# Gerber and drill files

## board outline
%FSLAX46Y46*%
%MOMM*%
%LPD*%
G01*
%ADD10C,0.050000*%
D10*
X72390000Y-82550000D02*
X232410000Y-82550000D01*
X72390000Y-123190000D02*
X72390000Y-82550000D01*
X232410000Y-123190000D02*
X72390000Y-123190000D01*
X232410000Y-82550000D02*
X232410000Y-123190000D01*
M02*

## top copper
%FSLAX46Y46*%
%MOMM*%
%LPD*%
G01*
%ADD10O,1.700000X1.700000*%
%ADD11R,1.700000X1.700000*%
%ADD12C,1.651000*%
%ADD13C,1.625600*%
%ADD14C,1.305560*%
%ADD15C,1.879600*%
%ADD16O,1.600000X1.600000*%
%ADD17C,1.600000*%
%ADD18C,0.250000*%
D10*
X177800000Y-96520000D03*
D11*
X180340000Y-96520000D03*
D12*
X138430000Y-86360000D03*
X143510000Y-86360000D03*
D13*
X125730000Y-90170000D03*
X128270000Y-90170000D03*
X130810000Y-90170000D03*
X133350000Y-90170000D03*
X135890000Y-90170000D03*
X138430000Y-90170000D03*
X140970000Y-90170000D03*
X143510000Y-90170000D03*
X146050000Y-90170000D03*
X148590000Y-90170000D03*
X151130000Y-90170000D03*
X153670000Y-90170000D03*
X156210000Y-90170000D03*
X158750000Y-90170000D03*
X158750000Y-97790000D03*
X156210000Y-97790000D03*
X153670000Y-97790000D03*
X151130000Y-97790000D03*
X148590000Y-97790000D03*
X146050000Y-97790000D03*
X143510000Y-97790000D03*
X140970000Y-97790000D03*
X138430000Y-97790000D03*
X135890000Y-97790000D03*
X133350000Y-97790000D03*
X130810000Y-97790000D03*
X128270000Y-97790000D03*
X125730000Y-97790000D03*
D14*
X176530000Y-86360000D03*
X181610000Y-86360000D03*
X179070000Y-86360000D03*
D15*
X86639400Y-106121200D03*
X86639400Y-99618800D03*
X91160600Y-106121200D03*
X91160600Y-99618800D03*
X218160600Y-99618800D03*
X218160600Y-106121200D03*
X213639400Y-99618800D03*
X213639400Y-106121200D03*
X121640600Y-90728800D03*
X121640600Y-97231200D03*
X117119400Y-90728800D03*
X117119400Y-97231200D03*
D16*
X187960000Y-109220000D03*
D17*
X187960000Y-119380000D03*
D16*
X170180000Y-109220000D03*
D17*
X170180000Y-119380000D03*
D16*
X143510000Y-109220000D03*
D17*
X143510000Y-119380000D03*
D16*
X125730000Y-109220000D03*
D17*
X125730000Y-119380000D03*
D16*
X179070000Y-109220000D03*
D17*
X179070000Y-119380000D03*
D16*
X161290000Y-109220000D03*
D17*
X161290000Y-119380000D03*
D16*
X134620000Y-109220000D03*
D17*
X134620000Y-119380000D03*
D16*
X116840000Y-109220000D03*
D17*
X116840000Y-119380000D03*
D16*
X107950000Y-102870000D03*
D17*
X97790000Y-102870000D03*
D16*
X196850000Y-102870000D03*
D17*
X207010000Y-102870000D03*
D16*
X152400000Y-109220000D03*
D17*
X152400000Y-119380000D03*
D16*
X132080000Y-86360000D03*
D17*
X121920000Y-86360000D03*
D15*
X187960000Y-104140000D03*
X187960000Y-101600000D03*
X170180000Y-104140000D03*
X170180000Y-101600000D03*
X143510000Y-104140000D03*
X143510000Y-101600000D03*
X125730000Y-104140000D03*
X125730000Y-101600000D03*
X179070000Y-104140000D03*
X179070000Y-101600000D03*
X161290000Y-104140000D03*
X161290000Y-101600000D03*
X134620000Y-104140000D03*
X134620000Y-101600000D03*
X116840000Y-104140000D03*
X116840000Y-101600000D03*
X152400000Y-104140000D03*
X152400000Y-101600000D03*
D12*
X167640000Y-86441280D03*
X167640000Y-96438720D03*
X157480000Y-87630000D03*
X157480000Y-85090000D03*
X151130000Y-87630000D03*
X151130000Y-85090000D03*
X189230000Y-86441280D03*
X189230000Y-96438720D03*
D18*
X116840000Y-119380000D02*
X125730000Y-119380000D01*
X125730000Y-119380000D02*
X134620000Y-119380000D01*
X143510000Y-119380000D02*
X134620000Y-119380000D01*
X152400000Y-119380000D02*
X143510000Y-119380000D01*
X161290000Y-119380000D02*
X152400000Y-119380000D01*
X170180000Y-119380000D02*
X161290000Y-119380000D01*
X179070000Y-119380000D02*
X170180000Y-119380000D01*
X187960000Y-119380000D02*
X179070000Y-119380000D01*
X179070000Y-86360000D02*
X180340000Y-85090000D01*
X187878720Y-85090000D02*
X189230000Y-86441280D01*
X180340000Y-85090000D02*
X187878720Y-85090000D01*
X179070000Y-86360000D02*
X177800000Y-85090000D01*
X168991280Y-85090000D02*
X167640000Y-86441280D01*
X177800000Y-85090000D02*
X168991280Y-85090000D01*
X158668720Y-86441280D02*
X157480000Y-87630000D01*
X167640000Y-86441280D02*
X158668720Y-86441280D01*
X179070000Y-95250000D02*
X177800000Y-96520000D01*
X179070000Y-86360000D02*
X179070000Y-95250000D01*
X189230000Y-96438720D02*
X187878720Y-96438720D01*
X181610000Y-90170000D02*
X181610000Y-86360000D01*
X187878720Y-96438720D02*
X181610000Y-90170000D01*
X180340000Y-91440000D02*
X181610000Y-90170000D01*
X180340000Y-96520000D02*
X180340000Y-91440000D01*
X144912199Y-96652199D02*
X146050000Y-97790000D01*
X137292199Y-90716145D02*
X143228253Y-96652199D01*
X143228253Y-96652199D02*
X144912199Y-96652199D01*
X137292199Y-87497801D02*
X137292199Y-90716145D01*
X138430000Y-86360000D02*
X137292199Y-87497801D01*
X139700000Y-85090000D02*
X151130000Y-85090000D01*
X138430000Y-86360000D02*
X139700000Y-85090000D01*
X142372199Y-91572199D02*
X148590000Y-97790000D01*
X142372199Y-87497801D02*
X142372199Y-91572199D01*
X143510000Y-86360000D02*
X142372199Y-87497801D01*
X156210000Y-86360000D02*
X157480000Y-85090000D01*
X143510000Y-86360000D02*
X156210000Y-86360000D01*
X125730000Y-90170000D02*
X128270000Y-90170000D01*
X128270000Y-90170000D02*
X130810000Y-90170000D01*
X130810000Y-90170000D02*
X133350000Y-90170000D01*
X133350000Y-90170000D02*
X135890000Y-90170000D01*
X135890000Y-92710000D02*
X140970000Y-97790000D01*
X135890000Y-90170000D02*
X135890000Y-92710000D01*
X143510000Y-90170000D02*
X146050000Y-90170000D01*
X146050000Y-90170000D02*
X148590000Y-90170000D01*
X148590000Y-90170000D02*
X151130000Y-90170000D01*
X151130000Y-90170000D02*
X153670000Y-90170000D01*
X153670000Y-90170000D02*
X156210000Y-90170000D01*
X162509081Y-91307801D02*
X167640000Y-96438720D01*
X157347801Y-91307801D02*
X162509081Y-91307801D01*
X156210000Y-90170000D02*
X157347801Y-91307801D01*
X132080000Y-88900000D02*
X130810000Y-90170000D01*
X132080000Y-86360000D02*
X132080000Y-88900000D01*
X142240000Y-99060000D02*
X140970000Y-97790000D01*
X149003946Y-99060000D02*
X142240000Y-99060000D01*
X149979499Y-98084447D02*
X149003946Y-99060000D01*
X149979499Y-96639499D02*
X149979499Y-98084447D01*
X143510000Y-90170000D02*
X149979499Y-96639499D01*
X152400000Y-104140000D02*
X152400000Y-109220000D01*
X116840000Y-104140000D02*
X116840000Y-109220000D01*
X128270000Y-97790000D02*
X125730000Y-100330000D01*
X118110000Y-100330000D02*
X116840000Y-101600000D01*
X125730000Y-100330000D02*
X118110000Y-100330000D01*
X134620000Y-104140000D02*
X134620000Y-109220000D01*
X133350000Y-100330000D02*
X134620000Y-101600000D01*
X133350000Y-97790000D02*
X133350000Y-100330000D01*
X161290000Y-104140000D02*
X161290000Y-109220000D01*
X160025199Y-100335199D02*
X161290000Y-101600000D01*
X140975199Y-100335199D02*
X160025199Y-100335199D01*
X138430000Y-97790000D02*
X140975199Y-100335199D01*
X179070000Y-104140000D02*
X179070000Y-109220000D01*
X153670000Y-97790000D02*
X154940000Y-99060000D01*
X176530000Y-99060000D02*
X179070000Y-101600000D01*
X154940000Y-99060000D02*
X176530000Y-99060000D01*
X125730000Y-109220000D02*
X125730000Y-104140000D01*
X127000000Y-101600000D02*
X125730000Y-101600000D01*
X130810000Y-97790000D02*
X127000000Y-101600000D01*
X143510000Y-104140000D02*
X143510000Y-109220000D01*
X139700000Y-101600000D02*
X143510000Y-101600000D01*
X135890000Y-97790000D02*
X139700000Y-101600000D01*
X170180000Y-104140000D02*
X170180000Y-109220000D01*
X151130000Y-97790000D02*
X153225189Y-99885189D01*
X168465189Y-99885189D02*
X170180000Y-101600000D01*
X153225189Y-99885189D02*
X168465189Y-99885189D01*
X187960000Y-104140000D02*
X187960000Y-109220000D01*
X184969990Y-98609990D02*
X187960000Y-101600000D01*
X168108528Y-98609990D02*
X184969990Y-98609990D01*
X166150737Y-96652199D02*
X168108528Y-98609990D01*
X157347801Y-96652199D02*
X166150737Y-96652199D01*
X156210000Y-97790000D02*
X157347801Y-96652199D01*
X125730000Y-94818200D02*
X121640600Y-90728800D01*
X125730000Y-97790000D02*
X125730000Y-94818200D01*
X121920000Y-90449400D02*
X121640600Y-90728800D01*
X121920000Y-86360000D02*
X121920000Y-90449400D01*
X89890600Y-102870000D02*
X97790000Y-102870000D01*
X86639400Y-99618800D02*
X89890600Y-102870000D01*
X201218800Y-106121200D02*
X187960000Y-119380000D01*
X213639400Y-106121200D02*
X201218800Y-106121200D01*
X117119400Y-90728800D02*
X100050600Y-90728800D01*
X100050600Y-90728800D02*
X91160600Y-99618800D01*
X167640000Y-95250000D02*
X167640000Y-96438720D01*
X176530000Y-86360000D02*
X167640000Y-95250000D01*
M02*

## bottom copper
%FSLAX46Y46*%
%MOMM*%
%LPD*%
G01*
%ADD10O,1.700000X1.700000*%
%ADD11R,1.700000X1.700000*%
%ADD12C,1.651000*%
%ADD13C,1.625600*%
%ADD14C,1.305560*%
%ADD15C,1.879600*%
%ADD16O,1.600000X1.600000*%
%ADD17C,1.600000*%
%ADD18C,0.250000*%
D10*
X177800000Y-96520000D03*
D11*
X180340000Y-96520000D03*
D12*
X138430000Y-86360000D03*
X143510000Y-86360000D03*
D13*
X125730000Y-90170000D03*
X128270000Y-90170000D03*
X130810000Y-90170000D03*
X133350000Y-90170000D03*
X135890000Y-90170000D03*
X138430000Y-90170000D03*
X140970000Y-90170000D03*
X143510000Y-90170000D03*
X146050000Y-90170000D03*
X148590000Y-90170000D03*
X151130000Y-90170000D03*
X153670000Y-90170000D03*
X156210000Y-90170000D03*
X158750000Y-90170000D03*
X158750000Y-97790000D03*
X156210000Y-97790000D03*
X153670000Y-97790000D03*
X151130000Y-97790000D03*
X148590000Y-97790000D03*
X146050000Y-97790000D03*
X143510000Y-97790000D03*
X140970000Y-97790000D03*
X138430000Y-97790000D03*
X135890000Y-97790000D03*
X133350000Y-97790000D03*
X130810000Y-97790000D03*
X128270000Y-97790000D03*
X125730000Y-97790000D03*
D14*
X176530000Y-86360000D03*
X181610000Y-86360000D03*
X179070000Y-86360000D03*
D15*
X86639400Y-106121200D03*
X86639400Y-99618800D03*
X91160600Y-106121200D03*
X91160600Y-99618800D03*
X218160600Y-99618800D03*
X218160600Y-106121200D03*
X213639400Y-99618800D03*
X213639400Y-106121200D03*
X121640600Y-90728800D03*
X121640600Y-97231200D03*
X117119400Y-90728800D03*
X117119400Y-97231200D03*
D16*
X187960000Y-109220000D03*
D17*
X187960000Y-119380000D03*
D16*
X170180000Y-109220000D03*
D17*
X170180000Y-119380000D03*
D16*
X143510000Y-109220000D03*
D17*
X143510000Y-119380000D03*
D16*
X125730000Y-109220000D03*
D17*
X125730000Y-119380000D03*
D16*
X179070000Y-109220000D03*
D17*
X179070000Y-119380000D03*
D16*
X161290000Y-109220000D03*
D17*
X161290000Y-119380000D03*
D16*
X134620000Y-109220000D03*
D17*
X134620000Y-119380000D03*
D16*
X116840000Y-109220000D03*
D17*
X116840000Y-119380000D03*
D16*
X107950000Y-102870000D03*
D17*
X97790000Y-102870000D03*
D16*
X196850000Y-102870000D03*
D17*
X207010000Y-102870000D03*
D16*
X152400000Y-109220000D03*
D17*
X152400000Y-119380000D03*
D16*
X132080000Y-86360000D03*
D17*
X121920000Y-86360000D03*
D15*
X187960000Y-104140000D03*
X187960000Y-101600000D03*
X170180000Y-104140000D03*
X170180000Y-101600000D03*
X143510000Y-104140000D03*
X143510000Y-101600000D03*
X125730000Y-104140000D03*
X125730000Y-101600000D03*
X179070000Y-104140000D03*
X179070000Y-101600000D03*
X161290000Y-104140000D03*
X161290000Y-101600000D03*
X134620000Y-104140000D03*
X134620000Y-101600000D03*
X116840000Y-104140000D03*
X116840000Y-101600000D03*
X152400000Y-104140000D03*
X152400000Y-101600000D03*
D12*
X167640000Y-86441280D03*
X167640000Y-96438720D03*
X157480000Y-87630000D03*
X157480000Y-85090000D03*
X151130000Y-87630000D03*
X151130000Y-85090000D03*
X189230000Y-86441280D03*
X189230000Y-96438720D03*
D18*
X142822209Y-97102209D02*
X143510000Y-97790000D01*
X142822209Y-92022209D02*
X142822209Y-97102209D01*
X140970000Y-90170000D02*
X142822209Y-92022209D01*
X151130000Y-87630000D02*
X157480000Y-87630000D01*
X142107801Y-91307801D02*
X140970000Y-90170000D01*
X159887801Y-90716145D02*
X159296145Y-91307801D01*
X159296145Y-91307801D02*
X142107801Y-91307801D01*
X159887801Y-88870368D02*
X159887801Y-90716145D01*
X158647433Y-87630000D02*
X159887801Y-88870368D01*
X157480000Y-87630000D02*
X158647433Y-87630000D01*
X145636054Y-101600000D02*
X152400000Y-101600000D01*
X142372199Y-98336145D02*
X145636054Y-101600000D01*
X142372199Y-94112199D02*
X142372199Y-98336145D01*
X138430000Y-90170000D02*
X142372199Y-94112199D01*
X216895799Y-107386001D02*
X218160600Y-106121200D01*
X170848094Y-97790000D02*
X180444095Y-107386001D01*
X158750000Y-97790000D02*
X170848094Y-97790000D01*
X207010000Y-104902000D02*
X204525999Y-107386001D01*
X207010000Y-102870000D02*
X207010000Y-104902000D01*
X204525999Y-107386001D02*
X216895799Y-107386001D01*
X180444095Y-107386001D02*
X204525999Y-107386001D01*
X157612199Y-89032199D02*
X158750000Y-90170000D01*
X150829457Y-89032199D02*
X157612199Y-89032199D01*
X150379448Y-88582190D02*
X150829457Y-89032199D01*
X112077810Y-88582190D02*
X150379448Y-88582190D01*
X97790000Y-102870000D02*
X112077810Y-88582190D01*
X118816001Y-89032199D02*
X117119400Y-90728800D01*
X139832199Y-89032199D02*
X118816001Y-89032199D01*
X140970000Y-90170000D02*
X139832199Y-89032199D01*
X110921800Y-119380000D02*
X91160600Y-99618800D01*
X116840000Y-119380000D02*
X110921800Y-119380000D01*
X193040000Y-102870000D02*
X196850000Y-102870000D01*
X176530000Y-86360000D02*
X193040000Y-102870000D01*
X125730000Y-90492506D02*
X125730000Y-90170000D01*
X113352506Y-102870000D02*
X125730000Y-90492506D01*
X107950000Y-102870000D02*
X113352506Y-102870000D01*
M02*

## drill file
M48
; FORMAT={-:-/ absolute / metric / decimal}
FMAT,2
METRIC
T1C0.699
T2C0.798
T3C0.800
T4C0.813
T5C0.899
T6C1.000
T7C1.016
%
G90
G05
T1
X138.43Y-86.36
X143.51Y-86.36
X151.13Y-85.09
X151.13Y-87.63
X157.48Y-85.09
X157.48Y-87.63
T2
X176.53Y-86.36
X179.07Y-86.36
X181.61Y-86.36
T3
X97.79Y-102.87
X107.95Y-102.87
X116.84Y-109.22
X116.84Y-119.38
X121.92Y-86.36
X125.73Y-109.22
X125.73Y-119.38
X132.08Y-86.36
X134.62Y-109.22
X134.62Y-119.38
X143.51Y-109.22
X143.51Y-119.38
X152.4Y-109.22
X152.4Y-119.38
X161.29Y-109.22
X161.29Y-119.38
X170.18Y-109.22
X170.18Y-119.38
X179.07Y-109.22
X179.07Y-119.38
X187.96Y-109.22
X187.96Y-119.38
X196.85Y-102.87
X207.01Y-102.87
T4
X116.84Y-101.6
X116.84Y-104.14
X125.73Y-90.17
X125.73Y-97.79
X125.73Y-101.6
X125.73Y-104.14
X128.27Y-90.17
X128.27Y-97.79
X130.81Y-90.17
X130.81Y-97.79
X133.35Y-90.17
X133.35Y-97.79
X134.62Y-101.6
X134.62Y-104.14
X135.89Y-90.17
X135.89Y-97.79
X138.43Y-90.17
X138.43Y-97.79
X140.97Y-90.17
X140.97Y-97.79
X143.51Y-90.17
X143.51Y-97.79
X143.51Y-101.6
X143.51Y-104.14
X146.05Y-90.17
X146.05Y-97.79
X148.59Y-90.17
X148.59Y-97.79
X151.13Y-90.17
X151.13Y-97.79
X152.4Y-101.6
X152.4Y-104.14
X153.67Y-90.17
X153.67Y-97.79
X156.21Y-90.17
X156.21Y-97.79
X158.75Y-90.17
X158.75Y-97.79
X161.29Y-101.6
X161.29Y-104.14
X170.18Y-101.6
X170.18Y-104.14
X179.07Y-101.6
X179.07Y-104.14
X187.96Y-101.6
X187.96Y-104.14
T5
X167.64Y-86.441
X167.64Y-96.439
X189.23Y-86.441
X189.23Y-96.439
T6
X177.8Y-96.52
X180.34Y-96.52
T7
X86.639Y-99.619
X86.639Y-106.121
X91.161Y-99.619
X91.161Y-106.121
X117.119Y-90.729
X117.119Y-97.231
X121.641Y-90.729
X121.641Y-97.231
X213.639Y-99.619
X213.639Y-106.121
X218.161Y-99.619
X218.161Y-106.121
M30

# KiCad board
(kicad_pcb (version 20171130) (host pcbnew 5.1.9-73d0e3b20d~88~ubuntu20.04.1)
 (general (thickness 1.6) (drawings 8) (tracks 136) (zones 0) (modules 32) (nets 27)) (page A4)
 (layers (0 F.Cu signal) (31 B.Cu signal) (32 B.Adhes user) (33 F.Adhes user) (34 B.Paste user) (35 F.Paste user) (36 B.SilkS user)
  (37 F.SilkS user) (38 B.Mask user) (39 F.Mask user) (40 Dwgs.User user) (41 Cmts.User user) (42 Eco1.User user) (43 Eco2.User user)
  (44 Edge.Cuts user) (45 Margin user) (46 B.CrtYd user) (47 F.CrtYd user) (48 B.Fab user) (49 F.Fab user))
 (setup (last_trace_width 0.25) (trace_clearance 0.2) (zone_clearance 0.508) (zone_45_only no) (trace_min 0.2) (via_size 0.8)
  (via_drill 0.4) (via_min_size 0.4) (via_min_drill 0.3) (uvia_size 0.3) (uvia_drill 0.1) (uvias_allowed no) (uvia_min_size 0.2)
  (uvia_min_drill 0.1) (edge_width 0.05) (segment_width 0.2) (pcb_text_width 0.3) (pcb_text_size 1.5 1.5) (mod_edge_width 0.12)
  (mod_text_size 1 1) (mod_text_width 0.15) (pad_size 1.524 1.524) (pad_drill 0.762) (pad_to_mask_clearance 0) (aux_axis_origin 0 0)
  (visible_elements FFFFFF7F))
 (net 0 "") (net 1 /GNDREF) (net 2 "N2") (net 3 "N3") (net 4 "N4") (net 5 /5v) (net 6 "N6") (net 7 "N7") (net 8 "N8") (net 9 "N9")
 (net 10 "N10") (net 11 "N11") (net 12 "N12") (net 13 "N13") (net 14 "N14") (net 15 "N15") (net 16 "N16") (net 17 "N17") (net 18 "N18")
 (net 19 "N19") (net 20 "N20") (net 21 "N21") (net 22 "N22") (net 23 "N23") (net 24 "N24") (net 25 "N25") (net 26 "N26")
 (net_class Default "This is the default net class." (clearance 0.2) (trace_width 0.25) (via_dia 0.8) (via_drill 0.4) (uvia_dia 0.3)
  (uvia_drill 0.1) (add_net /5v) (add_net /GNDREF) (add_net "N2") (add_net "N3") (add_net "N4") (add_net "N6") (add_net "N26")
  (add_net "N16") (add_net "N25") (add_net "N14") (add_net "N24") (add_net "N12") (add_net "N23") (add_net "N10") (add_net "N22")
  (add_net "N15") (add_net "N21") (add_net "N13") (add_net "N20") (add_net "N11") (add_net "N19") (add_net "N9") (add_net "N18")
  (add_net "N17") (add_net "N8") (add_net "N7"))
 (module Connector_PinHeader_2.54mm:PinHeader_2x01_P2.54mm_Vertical (layer F.Cu) (at 180.34 96.52 180)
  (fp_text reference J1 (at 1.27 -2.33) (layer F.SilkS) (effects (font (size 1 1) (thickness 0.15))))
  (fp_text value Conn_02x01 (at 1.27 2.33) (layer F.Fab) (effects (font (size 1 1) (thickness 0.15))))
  (pad 2 thru_hole oval (at 2.54 0 180) (size 1.7 1.7) (drill 1) (layers *.Cu *.Mask) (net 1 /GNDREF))
  (pad 1 thru_hole rect (at 0 0 180) (size 1.7 1.7) (drill 1) (layers *.Cu *.Mask) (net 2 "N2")))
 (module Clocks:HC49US (layer F.Cu) (at 140.97 86.36 180)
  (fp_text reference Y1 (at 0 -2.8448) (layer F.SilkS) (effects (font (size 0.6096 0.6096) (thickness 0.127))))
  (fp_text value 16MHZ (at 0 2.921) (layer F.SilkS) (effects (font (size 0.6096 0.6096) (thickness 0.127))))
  (pad 2 thru_hole circle (at 2.54 0 180) (size 1.651 1.651) (drill 0.6985) (layers *.Cu *.Mask) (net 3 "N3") (solder_mask_margin 0.1016))
  (pad 1 thru_hole circle (at -2.54 0 180) (size 1.651 1.651) (drill 0.6985) (layers *.Cu *.Mask) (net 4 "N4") (solder_mask_margin 0.1016)))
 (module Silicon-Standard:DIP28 (layer F.Cu) (at 142.24 93.98)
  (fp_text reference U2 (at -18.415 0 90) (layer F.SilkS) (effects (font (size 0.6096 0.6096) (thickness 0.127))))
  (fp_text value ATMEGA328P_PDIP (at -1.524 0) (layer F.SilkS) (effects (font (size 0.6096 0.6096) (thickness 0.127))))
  (pad 28 thru_hole circle (at -16.51 -3.81) (size 1.6256 1.6256) (drill 0.8128) (layers *.Cu *.Mask) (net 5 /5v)
   (solder_mask_margin 0.1016))
  (pad 27 thru_hole circle (at -13.97 -3.81) (size 1.6256 1.6256) (drill 0.8128) (layers *.Cu *.Mask) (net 5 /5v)
   (solder_mask_margin 0.1016))
  (pad 26 thru_hole circle (at -11.43 -3.81) (size 1.6256 1.6256) (drill 0.8128) (layers *.Cu *.Mask) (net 5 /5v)
   (solder_mask_margin 0.1016))
  (pad 25 thru_hole circle (at -8.89 -3.81) (size 1.6256 1.6256) (drill 0.8128) (layers *.Cu *.Mask) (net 5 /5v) (solder_mask_margin 0.1016))
  (pad 24 thru_hole circle (at -6.35 -3.81) (size 1.6256 1.6256) (drill 0.8128) (layers *.Cu *.Mask) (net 5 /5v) (solder_mask_margin 0.1016))
  (pad 23 thru_hole circle (at -3.81 -3.81) (size 1.6256 1.6256) (drill 0.8128) (layers *.Cu *.Mask) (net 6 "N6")
   (solder_mask_margin 0.1016))
  (pad 22 thru_hole circle (at -1.27 -3.81) (size 1.6256 1.6256) (drill 0.8128) (layers *.Cu *.Mask) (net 1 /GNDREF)
   (solder_mask_margin 0.1016))
  (pad 21 thru_hole circle (at 1.27 -3.81) (size 1.6256 1.6256) (drill 0.8128) (layers *.Cu *.Mask) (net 5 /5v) (solder_mask_margin 0.1016))
  (pad 20 thru_hole circle (at 3.81 -3.81) (size 1.6256 1.6256) (drill 0.8128) (layers *.Cu *.Mask) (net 5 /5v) (solder_mask_margin 0.1016))
  (pad 19 thru_hole circle (at 6.35 -3.81) (size 1.6256 1.6256) (drill 0.8128) (layers *.Cu *.Mask) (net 5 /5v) (solder_mask_margin 0.1016))
  (pad 18 thru_hole circle (at 8.89 -3.81) (size 1.6256 1.6256) (drill 0.8128) (layers *.Cu *.Mask) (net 5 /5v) (solder_mask_margin 0.1016))
  (pad 17 thru_hole circle (at 11.43 -3.81) (size 1.6256 1.6256) (drill 0.8128) (layers *.Cu *.Mask) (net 5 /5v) (solder_mask_margin 0.1016))
  (pad 16 thru_hole circle (at 13.97 -3.81) (size 1.6256 1.6256) (drill 0.8128) (layers *.Cu *.Mask) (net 5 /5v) (solder_mask_margin 0.1016))
  (pad 15 thru_hole circle (at 16.51 -3.81) (size 1.6256 1.6256) (drill 0.8128) (layers *.Cu *.Mask) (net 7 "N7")
   (solder_mask_margin 0.1016))
  (pad 14 thru_hole circle (at 16.51 3.81) (size 1.6256 1.6256) (drill 0.8128) (layers *.Cu *.Mask) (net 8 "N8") (solder_mask_margin 0.1016))
  (pad 13 thru_hole circle (at 13.97 3.81) (size 1.6256 1.6256) (drill 0.8128) (layers *.Cu *.Mask) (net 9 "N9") (solder_mask_margin 0.1016))
  (pad 12 thru_hole circle (at 11.43 3.81) (size 1.6256 1.6256) (drill 0.8128) (layers *.Cu *.Mask) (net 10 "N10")
   (solder_mask_margin 0.1016))
  (pad 11 thru_hole circle (at 8.89 3.81) (size 1.6256 1.6256) (drill 0.8128) (layers *.Cu *.Mask) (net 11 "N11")
   (solder_mask_margin 0.1016))
  (pad 10 thru_hole circle (at 6.35 3.81) (size 1.6256 1.6256) (drill 0.8128) (layers *.Cu *.Mask) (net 4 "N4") (solder_mask_margin 0.1016))
  (pad 9 thru_hole circle (at 3.81 3.81) (size 1.6256 1.6256) (drill 0.8128) (layers *.Cu *.Mask) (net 3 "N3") (solder_mask_margin 0.1016))
  (pad 8 thru_hole circle (at 1.27 3.81) (size 1.6256 1.6256) (drill 0.8128) (layers *.Cu *.Mask) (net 1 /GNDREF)
   (solder_mask_margin 0.1016))
  (pad 7 thru_hole circle (at -1.27 3.81) (size 1.6256 1.6256) (drill 0.8128) (layers *.Cu *.Mask) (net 5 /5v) (solder_mask_margin 0.1016))
  (pad 6 thru_hole circle (at -3.81 3.81) (size 1.6256 1.6256) (drill 0.8128) (layers *.Cu *.Mask) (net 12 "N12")
   (solder_mask_margin 0.1016))
  (pad 5 thru_hole circle (at -6.35 3.81) (size 1.6256 1.6256) (drill 0.8128) (layers *.Cu *.Mask) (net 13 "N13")
   (solder_mask_margin 0.1016))
  (pad 4 thru_hole circle (at -8.89 3.81) (size 1.6256 1.6256) (drill 0.8128) (layers *.Cu *.Mask) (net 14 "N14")
   (solder_mask_margin 0.1016))
  (pad 3 thru_hole circle (at -11.43 3.81) (size 1.6256 1.6256) (drill 0.8128) (layers *.Cu *.Mask) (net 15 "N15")
   (solder_mask_margin 0.1016))
  (pad 2 thru_hole circle (at -13.97 3.81) (size 1.6256 1.6256) (drill 0.8128) (layers *.Cu *.Mask) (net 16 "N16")
   (solder_mask_margin 0.1016))
  (pad 1 thru_hole circle (at -16.51 3.81) (size 1.6256 1.6256) (drill 0.8128) (layers *.Cu *.Mask) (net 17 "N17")
   (solder_mask_margin 0.1016)))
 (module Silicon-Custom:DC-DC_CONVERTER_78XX (layer F.Cu) (at 179.07 86.36 180)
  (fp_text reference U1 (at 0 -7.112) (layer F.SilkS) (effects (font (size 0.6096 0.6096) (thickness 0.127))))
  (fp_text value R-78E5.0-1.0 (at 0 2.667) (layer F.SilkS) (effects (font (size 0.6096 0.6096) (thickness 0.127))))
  (pad VOUT thru_hole circle (at 2.54 0 180) (size 1.30556 1.30556) (drill 0.79756) (layers *.Cu *.Mask) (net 5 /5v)
   (solder_mask_margin 0.1016))
  (pad VIN thru_hole circle (at -2.54 0 180) (size 1.30556 1.30556) (drill 0.79756) (layers *.Cu *.Mask) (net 2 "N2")
   (solder_mask_margin 0.1016))
  (pad GND thru_hole circle (at 0 0 180) (size 1.30556 1.30556) (drill 0.79756) (layers *.Cu *.Mask) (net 1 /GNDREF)
   (solder_mask_margin 0.1016)))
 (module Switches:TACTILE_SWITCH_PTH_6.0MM (layer F.Cu) (at 88.9 102.87 270)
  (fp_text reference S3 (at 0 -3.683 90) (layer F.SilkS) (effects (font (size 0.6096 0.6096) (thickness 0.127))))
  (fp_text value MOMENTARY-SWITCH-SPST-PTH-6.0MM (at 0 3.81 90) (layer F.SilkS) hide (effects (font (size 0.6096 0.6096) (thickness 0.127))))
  (pad 4 thru_hole circle (at 3.2512 2.2606 270) (size 1.8796 1.8796) (drill 1.016) (layers *.Cu *.Mask) (solder_mask_margin 0.1016))
  (pad 3 thru_hole circle (at -3.2512 2.2606 270) (size 1.8796 1.8796) (drill 1.016) (layers *.Cu *.Mask) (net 7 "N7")
   (solder_mask_margin 0.1016))
  (pad 2 thru_hole circle (at 3.2512 -2.2606 270) (size 1.8796 1.8796) (drill 1.016) (layers *.Cu *.Mask) (solder_mask_margin 0.1016))
  (pad 1 thru_hole circle (at -3.2512 -2.2606 270) (size 1.8796 1.8796) (drill 1.016) (layers *.Cu *.Mask) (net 1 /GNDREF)
   (solder_mask_margin 0.1016)))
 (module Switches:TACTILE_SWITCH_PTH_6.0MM (layer F.Cu) (at 215.9 102.87 90)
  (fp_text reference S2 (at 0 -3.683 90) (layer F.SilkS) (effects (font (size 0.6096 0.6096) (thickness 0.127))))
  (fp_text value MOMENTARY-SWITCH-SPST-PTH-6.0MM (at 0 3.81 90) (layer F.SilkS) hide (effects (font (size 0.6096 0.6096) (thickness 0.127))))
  (pad 4 thru_hole circle (at 3.2512 2.2606 90) (size 1.8796 1.8796) (drill 1.016) (layers *.Cu *.Mask) (solder_mask_margin 0.1016))
  (pad 3 thru_hole circle (at -3.2512 2.2606 90) (size 1.8796 1.8796) (drill 1.016) (layers *.Cu *.Mask) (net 8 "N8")
   (solder_mask_margin 0.1016))
  (pad 2 thru_hole circle (at 3.2512 -2.2606 90) (size 1.8796 1.8796) (drill 1.016) (layers *.Cu *.Mask) (solder_mask_margin 0.1016))
  (pad 1 thru_hole circle (at -3.2512 -2.2606 90) (size 1.8796 1.8796) (drill 1.016) (layers *.Cu *.Mask) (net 1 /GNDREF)
   (solder_mask_margin 0.1016)))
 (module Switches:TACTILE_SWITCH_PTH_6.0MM (layer F.Cu) (at 119.38 93.98 270)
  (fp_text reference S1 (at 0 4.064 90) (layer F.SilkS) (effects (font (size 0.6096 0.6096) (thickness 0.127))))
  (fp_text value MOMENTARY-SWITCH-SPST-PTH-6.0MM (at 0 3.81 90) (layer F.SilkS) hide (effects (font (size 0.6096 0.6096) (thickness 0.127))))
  (pad 1 thru_hole circle (at -3.2512 -2.2606 270) (size 1.8796 1.8796) (drill 1.016) (layers *.Cu *.Mask) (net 17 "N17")
   (solder_mask_margin 0.1016))
  (pad 2 thru_hole circle (at 3.2512 -2.2606 270) (size 1.8796 1.8796) (drill 1.016) (layers *.Cu *.Mask) (solder_mask_margin 0.1016))
  (pad 3 thru_hole circle (at -3.2512 2.2606 270) (size 1.8796 1.8796) (drill 1.016) (layers *.Cu *.Mask) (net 1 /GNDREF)
   (solder_mask_margin 0.1016))
  (pad 4 thru_hole circle (at 3.2512 2.2606 270) (size 1.8796 1.8796) (drill 1.016) (layers *.Cu *.Mask) (solder_mask_margin 0.1016)))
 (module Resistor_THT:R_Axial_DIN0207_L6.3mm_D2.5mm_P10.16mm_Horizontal (layer F.Cu) (at 187.96 119.38 90)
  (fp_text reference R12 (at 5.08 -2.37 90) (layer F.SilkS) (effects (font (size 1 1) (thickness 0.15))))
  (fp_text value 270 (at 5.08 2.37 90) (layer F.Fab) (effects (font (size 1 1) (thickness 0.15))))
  (pad 2 thru_hole oval (at 10.16 0 90) (size 1.6 1.6) (drill 0.8) (layers *.Cu *.Mask) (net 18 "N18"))
  (pad 1 thru_hole circle (at 0 0 90) (size 1.6 1.6) (drill 0.8) (layers *.Cu *.Mask) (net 1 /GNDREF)))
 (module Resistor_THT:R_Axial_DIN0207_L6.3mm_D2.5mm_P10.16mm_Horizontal (layer F.Cu) (at 170.18 119.38 90)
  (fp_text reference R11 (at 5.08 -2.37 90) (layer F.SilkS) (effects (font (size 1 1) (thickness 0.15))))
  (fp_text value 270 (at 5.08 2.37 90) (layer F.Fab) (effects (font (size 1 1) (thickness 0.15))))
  (pad 2 thru_hole oval (at 10.16 0 90) (size 1.6 1.6) (drill 0.8) (layers *.Cu *.Mask) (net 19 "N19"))
  (pad 1 thru_hole circle (at 0 0 90) (size 1.6 1.6) (drill 0.8) (layers *.Cu *.Mask) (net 1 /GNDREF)))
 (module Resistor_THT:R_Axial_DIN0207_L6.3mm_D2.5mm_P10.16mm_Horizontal (layer F.Cu) (at 143.51 119.38 90)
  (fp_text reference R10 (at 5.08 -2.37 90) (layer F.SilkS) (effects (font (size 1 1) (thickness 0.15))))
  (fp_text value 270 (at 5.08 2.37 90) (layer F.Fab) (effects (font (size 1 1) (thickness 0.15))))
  (pad 2 thru_hole oval (at 10.16 0 90) (size 1.6 1.6) (drill 0.8) (layers *.Cu *.Mask) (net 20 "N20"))
  (pad 1 thru_hole circle (at 0 0 90) (size 1.6 1.6) (drill 0.8) (layers *.Cu *.Mask) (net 1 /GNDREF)))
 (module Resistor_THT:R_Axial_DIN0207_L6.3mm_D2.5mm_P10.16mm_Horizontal (layer F.Cu) (at 125.73 119.38 90)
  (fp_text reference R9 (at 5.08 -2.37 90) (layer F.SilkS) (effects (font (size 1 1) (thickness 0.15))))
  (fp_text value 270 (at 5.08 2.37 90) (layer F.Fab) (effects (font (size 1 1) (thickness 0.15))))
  (pad 2 thru_hole oval (at 10.16 0 90) (size 1.6 1.6) (drill 0.8) (layers *.Cu *.Mask) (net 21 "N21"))
  (pad 1 thru_hole circle (at 0 0 90) (size 1.6 1.6) (drill 0.8) (layers *.Cu *.Mask) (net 1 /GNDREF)))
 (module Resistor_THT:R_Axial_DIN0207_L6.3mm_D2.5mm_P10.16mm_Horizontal (layer F.Cu) (at 179.07 119.38 90)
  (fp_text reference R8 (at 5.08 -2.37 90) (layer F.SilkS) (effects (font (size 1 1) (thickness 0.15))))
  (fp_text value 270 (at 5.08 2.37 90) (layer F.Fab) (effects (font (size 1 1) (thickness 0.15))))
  (pad 2 thru_hole oval (at 10.16 0 90) (size 1.6 1.6) (drill 0.8) (layers *.Cu *.Mask) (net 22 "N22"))
  (pad 1 thru_hole circle (at 0 0 90) (size 1.6 1.6) (drill 0.8) (layers *.Cu *.Mask) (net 1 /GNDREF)))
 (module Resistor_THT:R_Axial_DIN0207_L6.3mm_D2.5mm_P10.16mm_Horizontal (layer F.Cu) (at 161.29 119.38 90)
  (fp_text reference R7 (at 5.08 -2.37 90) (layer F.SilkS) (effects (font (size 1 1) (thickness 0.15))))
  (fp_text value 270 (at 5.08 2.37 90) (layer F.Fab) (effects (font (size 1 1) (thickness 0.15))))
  (pad 2 thru_hole oval (at 10.16 0 90) (size 1.6 1.6) (drill 0.8) (layers *.Cu *.Mask) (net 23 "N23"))
  (pad 1 thru_hole circle (at 0 0 90) (size 1.6 1.6) (drill 0.8) (layers *.Cu *.Mask) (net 1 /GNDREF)))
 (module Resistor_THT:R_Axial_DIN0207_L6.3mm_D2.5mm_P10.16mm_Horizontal (layer F.Cu) (at 134.62 119.38 90)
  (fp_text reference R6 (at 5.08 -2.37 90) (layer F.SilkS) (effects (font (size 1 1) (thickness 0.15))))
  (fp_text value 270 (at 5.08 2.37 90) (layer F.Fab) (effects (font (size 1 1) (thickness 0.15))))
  (pad 2 thru_hole oval (at 10.16 0 90) (size 1.6 1.6) (drill 0.8) (layers *.Cu *.Mask) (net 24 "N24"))
  (pad 1 thru_hole circle (at 0 0 90) (size 1.6 1.6) (drill 0.8) (layers *.Cu *.Mask) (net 1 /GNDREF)))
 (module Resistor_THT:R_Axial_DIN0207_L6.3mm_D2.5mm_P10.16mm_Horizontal (layer F.Cu) (at 116.84 119.38 90)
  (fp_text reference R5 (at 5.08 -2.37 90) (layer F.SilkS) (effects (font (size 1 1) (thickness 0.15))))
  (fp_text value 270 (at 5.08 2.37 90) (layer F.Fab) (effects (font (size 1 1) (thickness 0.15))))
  (pad 2 thru_hole oval (at 10.16 0 90) (size 1.6 1.6) (drill 0.8) (layers *.Cu *.Mask) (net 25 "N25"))
  (pad 1 thru_hole circle (at 0 0 90) (size 1.6 1.6) (drill 0.8) (layers *.Cu *.Mask) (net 1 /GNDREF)))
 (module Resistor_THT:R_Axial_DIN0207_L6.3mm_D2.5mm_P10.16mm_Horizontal (layer F.Cu) (at 97.79 102.87)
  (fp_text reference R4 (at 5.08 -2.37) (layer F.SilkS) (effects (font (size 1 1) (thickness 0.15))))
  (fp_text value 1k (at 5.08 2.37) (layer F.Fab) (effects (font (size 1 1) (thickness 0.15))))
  (pad 2 thru_hole oval (at 10.16 0) (size 1.6 1.6) (drill 0.8) (layers *.Cu *.Mask) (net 5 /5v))
  (pad 1 thru_hole circle (at 0 0) (size 1.6 1.6) (drill 0.8) (layers *.Cu *.Mask) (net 7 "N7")))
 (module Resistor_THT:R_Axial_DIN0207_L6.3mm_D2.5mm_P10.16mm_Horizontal (layer F.Cu) (at 207.01 102.87 180)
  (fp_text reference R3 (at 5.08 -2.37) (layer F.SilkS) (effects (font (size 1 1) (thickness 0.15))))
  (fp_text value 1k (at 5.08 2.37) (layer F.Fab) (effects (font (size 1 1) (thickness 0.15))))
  (pad 2 thru_hole oval (at 10.16 0 180) (size 1.6 1.6) (drill 0.8) (layers *.Cu *.Mask) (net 5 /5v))
  (pad 1 thru_hole circle (at 0 0 180) (size 1.6 1.6) (drill 0.8) (layers *.Cu *.Mask) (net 8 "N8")))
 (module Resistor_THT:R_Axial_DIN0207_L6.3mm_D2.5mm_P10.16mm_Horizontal (layer F.Cu) (at 152.4 119.38 90)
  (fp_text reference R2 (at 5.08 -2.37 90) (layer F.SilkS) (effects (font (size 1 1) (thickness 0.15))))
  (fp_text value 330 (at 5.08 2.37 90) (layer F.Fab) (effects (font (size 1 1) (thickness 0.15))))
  (pad 2 thru_hole oval (at 10.16 0 90) (size 1.6 1.6) (drill 0.8) (layers *.Cu *.Mask) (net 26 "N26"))
  (pad 1 thru_hole circle (at 0 0 90) (size 1.6 1.6) (drill 0.8) (layers *.Cu *.Mask) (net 1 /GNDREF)))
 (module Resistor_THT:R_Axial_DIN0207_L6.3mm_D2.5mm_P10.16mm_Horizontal (layer F.Cu) (at 121.92 86.36)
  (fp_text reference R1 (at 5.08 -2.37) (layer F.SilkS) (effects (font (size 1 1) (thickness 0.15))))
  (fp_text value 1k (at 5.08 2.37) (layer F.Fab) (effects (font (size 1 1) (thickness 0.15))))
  (pad 2 thru_hole oval (at 10.16 0) (size 1.6 1.6) (drill 0.8) (layers *.Cu *.Mask) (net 5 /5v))
  (pad 1 thru_hole circle (at 0 0) (size 1.6 1.6) (drill 0.8) (layers *.Cu *.Mask) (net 17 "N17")))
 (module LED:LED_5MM (layer F.Cu) (at 187.96 102.87 270)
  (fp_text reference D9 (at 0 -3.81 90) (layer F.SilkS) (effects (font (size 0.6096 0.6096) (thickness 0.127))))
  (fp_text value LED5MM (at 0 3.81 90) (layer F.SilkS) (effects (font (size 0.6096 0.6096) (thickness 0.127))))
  (pad K thru_hole circle (at 1.27 0 270) (size 1.8796 1.8796) (drill 0.8128) (layers *.Cu *.Mask) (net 18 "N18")
   (solder_mask_margin 0.1016))
  (pad A thru_hole circle (at -1.27 0 270) (size 1.8796 1.8796) (drill 0.8128) (layers *.Cu *.Mask) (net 9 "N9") (solder_mask_margin 0.1016)))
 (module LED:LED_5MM (layer F.Cu) (at 170.18 102.87 270)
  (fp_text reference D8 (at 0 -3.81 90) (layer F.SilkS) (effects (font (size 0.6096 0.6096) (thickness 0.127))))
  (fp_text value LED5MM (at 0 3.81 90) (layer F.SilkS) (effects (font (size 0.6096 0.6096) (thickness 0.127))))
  (pad K thru_hole circle (at 1.27 0 270) (size 1.8796 1.8796) (drill 0.8128) (layers *.Cu *.Mask) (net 19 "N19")
   (solder_mask_margin 0.1016))
  (pad A thru_hole circle (at -1.27 0 270) (size 1.8796 1.8796) (drill 0.8128) (layers *.Cu *.Mask) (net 11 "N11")
   (solder_mask_margin 0.1016)))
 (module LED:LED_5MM (layer F.Cu) (at 143.51 102.87 270)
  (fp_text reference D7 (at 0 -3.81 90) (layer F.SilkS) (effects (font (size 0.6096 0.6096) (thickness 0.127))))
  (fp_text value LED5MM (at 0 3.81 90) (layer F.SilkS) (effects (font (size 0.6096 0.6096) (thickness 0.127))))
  (pad K thru_hole circle (at 1.27 0 270) (size 1.8796 1.8796) (drill 0.8128) (layers *.Cu *.Mask) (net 20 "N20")
   (solder_mask_margin 0.1016))
  (pad A thru_hole circle (at -1.27 0 270) (size 1.8796 1.8796) (drill 0.8128) (layers *.Cu *.Mask) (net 13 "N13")
   (solder_mask_margin 0.1016)))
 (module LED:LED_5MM (layer F.Cu) (at 125.73 102.87 270)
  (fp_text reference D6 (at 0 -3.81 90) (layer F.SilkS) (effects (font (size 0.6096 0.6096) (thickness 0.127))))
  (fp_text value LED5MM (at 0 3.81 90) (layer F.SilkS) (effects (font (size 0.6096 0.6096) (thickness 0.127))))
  (pad K thru_hole circle (at 1.27 0 270) (size 1.8796 1.8796) (drill 0.8128) (layers *.Cu *.Mask) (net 21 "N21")
   (solder_mask_margin 0.1016))
  (pad A thru_hole circle (at -1.27 0 270) (size 1.8796 1.8796) (drill 0.8128) (layers *.Cu *.Mask) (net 15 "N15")
   (solder_mask_margin 0.1016)))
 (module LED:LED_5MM (layer F.Cu) (at 179.07 102.87 270)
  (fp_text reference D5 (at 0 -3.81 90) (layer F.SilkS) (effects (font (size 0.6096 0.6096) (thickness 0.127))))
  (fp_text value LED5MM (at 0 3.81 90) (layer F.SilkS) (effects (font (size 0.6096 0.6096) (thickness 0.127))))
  (pad K thru_hole circle (at 1.27 0 270) (size 1.8796 1.8796) (drill 0.8128) (layers *.Cu *.Mask) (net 22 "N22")
   (solder_mask_margin 0.1016))
  (pad A thru_hole circle (at -1.27 0 270) (size 1.8796 1.8796) (drill 0.8128) (layers *.Cu *.Mask) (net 10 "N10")
   (solder_mask_margin 0.1016)))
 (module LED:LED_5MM (layer F.Cu) (at 161.29 102.87 270)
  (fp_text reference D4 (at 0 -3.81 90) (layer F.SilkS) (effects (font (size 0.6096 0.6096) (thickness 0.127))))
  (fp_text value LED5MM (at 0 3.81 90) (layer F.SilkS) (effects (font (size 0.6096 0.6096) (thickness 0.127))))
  (pad K thru_hole circle (at 1.27 0 270) (size 1.8796 1.8796) (drill 0.8128) (layers *.Cu *.Mask) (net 23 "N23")
   (solder_mask_margin 0.1016))
  (pad A thru_hole circle (at -1.27 0 270) (size 1.8796 1.8796) (drill 0.8128) (layers *.Cu *.Mask) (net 12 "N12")
   (solder_mask_margin 0.1016)))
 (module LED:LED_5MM (layer F.Cu) (at 134.62 102.87 270)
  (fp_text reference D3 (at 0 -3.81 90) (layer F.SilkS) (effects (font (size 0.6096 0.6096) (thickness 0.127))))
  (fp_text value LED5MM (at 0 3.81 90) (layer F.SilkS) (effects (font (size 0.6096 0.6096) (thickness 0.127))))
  (pad K thru_hole circle (at 1.27 0 270) (size 1.8796 1.8796) (drill 0.8128) (layers *.Cu *.Mask) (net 24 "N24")
   (solder_mask_margin 0.1016))
  (pad A thru_hole circle (at -1.27 0 270) (size 1.8796 1.8796) (drill 0.8128) (layers *.Cu *.Mask) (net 14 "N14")
   (solder_mask_margin 0.1016)))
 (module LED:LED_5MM (layer F.Cu) (at 116.84 102.87 270)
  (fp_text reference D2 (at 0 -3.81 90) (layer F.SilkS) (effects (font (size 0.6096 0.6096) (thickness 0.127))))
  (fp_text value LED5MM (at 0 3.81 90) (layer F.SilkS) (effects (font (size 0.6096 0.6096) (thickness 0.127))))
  (pad K thru_hole circle (at 1.27 0 270) (size 1.8796 1.8796) (drill 0.8128) (layers *.Cu *.Mask) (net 25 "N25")
   (solder_mask_margin 0.1016))
  (pad A thru_hole circle (at -1.27 0 270) (size 1.8796 1.8796) (drill 0.8128) (layers *.Cu *.Mask) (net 16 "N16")
   (solder_mask_margin 0.1016)))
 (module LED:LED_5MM (layer F.Cu) (at 152.4 102.87 270)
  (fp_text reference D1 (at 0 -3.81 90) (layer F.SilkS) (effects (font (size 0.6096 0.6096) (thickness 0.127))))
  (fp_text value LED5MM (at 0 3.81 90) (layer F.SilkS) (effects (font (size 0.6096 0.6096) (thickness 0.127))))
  (pad K thru_hole circle (at 1.27 0 270) (size 1.8796 1.8796) (drill 0.8128) (layers *.Cu *.Mask) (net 26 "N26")
   (solder_mask_margin 0.1016))
  (pad A thru_hole circle (at -1.27 0 270) (size 1.8796 1.8796) (drill 0.8128) (layers *.Cu *.Mask) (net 6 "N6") (solder_mask_margin 0.1016)))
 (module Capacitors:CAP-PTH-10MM (layer F.Cu) (at 167.64 91.44 90)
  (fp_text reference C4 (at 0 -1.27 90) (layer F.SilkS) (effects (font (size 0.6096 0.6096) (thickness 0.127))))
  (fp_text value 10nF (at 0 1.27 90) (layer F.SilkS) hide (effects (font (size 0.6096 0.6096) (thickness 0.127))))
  (pad 2 thru_hole circle (at 4.99872 0 90) (size 1.651 1.651) (drill 0.89916) (layers *.Cu *.Mask) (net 1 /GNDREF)
   (solder_mask_margin 0.1016))
  (pad 1 thru_hole circle (at -4.99872 0 90) (size 1.651 1.651) (drill 0.89916) (layers *.Cu *.Mask) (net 5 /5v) (solder_mask_margin 0.1016)))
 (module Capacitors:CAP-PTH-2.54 (layer F.Cu) (at 157.48 86.36 270)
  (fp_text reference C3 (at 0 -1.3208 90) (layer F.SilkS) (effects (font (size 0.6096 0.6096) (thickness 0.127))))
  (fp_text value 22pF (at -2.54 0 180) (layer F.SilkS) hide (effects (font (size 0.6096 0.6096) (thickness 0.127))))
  (pad 2 thru_hole circle (at 1.27 0 270) (size 1.651 1.651) (drill 0.6985) (layers *.Cu *.Mask) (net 1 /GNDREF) (solder_mask_margin 0.1016))
  (pad 1 thru_hole circle (at -1.27 0 270) (size 1.651 1.651) (drill 0.6985) (layers *.Cu *.Mask) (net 4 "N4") (solder_mask_margin 0.1016)))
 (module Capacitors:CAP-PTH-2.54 (layer F.Cu) (at 151.13 86.36 270)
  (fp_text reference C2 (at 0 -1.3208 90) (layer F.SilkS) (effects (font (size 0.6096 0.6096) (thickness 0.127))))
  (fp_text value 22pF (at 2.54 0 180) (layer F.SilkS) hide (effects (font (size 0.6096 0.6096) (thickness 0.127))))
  (pad 2 thru_hole circle (at 1.27 0 270) (size 1.651 1.651) (drill 0.6985) (layers *.Cu *.Mask) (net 1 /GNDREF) (solder_mask_margin 0.1016))
  (pad 1 thru_hole circle (at -1.27 0 270) (size 1.651 1.651) (drill 0.6985) (layers *.Cu *.Mask) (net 3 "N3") (solder_mask_margin 0.1016)))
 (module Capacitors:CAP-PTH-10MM (layer F.Cu) (at 189.23 91.44 90)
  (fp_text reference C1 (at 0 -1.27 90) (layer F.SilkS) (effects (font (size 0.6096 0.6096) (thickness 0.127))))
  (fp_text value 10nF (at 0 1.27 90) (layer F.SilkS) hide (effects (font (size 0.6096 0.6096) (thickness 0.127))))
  (pad 2 thru_hole circle (at 4.99872 0 90) (size 1.651 1.651) (drill 0.89916) (layers *.Cu *.Mask) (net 1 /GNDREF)
   (solder_mask_margin 0.1016))
  (pad 1 thru_hole circle (at -4.99872 0 90) (size 1.651 1.651) (drill 0.89916) (layers *.Cu *.Mask) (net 2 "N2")
   (solder_mask_margin 0.1016)))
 (gr_line (start 72.39 82.55) (end 232.41 82.55) (layer Edge.Cuts) (width 0.05))
 (gr_line (start 72.39 123.19) (end 72.39 82.55) (layer Edge.Cuts) (width 0.05))
 (gr_line (start 232.41 123.19) (end 72.39 123.19) (layer Edge.Cuts) (width 0.05))
 (gr_line (start 232.41 82.55) (end 232.41 123.19) (layer Edge.Cuts) (width 0.05))
 (segment (start 116.84 119.38) (end 125.73 119.38) (width 0.25) (layer F.Cu) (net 1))
 (segment (start 125.73 119.38) (end 134.62 119.38) (width 0.25) (layer F.Cu) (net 1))
 (segment (start 143.51 119.38) (end 134.62 119.38) (width 0.25) (layer F.Cu) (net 1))
 (segment (start 152.4 119.38) (end 143.51 119.38) (width 0.25) (layer F.Cu) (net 1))
 (segment (start 161.29 119.38) (end 152.4 119.38) (width 0.25) (layer F.Cu) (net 1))
 (segment (start 170.18 119.38) (end 161.29 119.38) (width 0.25) (layer F.Cu) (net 1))
 (segment (start 179.07 119.38) (end 170.18 119.38) (width 0.25) (layer F.Cu) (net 1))
 (segment (start 187.96 119.38) (end 179.07 119.38) (width 0.25) (layer F.Cu) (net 1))
 (segment (start 179.07 86.36) (end 180.34 85.09) (width 0.25) (layer F.Cu) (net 1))
 (segment (start 187.87872 85.09) (end 189.23 86.44128) (width 0.25) (layer F.Cu) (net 1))
 (segment (start 180.34 85.09) (end 187.87872 85.09) (width 0.25) (layer F.Cu) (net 1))
 (segment (start 179.07 86.36) (end 177.8 85.09) (width 0.25) (layer F.Cu) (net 1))
 (segment (start 168.99128 85.09) (end 167.64 86.44128) (width 0.25) (layer F.Cu) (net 1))
 (segment (start 177.8 85.09) (end 168.99128 85.09) (width 0.25) (layer F.Cu) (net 1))
 (segment (start 158.66872 86.44128) (end 157.48 87.63) (width 0.25) (layer F.Cu) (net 1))
 (segment (start 167.64 86.44128) (end 158.66872 86.44128) (width 0.25) (layer F.Cu) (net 1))
 (segment (start 142.822209 97.102209) (end 143.51 97.79) (width 0.25) (layer B.Cu) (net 1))
 (segment (start 142.822209 92.022209) (end 142.822209 97.102209) (width 0.25) (layer B.Cu) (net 1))
 (segment (start 140.97 90.17) (end 142.822209 92.022209) (width 0.25) (layer B.Cu) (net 1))
 (segment (start 151.13 87.63) (end 157.48 87.63) (width 0.25) (layer B.Cu) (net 1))
 (segment (start 142.107801 91.307801) (end 140.97 90.17) (width 0.25) (layer B.Cu) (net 1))
 (segment (start 159.887801 90.716145) (end 159.296145 91.307801) (width 0.25) (layer B.Cu) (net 1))
 (segment (start 159.296145 91.307801) (end 142.107801 91.307801) (width 0.25) (layer B.Cu) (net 1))
 (segment (start 159.887801 88.870368) (end 159.887801 90.716145) (width 0.25) (layer B.Cu) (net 1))
 (segment (start 158.647433 87.63) (end 159.887801 88.870368) (width 0.25) (layer B.Cu) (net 1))
 (segment (start 157.48 87.63) (end 158.647433 87.63) (width 0.25) (layer B.Cu) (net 1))
 (segment (start 179.07 95.25) (end 177.8 96.52) (width 0.25) (layer F.Cu) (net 1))
 (segment (start 179.07 86.36) (end 179.07 95.25) (width 0.25) (layer F.Cu) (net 1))
 (segment (start 189.23 96.43872) (end 187.87872 96.43872) (width 0.25) (layer F.Cu) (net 2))
 (segment (start 181.61 90.17) (end 181.61 86.36) (width 0.25) (layer F.Cu) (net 2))
 (segment (start 187.87872 96.43872) (end 181.61 90.17) (width 0.25) (layer F.Cu) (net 2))
 (segment (start 180.34 91.44) (end 181.61 90.17) (width 0.25) (layer F.Cu) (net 2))
 (segment (start 180.34 96.52) (end 180.34 91.44) (width 0.25) (layer F.Cu) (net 2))
 (segment (start 144.912199 96.652199) (end 146.05 97.79) (width 0.25) (layer F.Cu) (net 3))
 (segment (start 137.292199 90.716145) (end 143.228253 96.652199) (width 0.25) (layer F.Cu) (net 3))
 (segment (start 143.228253 96.652199) (end 144.912199 96.652199) (width 0.25) (layer F.Cu) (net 3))
 (segment (start 137.292199 87.497801) (end 137.292199 90.716145) (width 0.25) (layer F.Cu) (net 3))
 (segment (start 138.43 86.36) (end 137.292199 87.497801) (width 0.25) (layer F.Cu) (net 3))
 (segment (start 139.7 85.09) (end 151.13 85.09) (width 0.25) (layer F.Cu) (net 3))
 (segment (start 138.43 86.36) (end 139.7 85.09) (width 0.25) (layer F.Cu) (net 3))
 (segment (start 142.372199 91.572199) (end 148.59 97.79) (width 0.25) (layer F.Cu) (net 4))
 (segment (start 142.372199 87.497801) (end 142.372199 91.572199) (width 0.25) (layer F.Cu) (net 4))
 (segment (start 143.51 86.36) (end 142.372199 87.497801) (width 0.25) (layer F.Cu) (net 4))
 (segment (start 156.21 86.36) (end 157.48 85.09) (width 0.25) (layer F.Cu) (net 4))
 (segment (start 143.51 86.36) (end 156.21 86.36) (width 0.25) (layer F.Cu) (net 4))
 (segment (start 125.73 90.17) (end 128.27 90.17) (width 0.25) (layer F.Cu) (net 5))
 (segment (start 128.27 90.17) (end 130.81 90.17) (width 0.25) (layer F.Cu) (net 5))
 (segment (start 130.81 90.17) (end 133.35 90.17) (width 0.25) (layer F.Cu) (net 5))
 (segment (start 133.35 90.17) (end 135.89 90.17) (width 0.25) (layer F.Cu) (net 5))
 (segment (start 135.89 92.71) (end 140.97 97.79) (width 0.25) (layer F.Cu) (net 5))
 (segment (start 135.89 90.17) (end 135.89 92.71) (width 0.25) (layer F.Cu) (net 5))
 (segment (start 143.51 90.17) (end 146.05 90.17) (width 0.25) (layer F.Cu) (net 5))
 (segment (start 146.05 90.17) (end 148.59 90.17) (width 0.25) (layer F.Cu) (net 5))
 (segment (start 148.59 90.17) (end 151.13 90.17) (width 0.25) (layer F.Cu) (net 5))
 (segment (start 151.13 90.17) (end 153.67 90.17) (width 0.25) (layer F.Cu) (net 5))
 (segment (start 153.67 90.17) (end 156.21 90.17) (width 0.25) (layer F.Cu) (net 5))
 (segment (start 162.509081 91.307801) (end 167.64 96.43872) (width 0.25) (layer F.Cu) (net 5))
 (segment (start 157.347801 91.307801) (end 162.509081 91.307801) (width 0.25) (layer F.Cu) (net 5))
 (segment (start 156.21 90.17) (end 157.347801 91.307801) (width 0.25) (layer F.Cu) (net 5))
 (segment (start 132.08 88.9) (end 130.81 90.17) (width 0.25) (layer F.Cu) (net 5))
 (segment (start 132.08 86.36) (end 132.08 88.9) (width 0.25) (layer F.Cu) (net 5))
 (segment (start 142.24 99.06) (end 140.97 97.79) (width 0.25) (layer F.Cu) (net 5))
 (segment (start 149.003946 99.06) (end 142.24 99.06) (width 0.25) (layer F.Cu) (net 5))
 (segment (start 149.979499 98.084447) (end 149.003946 99.06) (width 0.25) (layer F.Cu) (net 5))
 (segment (start 149.979499 96.639499) (end 149.979499 98.084447) (width 0.25) (layer F.Cu) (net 5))
 (segment (start 143.51 90.17) (end 149.979499 96.639499) (width 0.25) (layer F.Cu) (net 5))
 (segment (start 152.4 104.14) (end 152.4 109.22) (width 0.25) (layer F.Cu) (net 26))
 (segment (start 145.636054 101.6) (end 152.4 101.6) (width 0.25) (layer B.Cu) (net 6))
 (segment (start 142.372199 98.336145) (end 145.636054 101.6) (width 0.25) (layer B.Cu) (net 6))
 (segment (start 142.372199 94.112199) (end 142.372199 98.336145) (width 0.25) (layer B.Cu) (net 6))
 (segment (start 138.43 90.17) (end 142.372199 94.112199) (width 0.25) (layer B.Cu) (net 6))
 (segment (start 116.84 104.14) (end 116.84 109.22) (width 0.25) (layer F.Cu) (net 25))
 (segment (start 128.27 97.79) (end 125.73 100.33) (width 0.25) (layer F.Cu) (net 16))
 (segment (start 118.11 100.33) (end 116.84 101.6) (width 0.25) (layer F.Cu) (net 16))
 (segment (start 125.73 100.33) (end 118.11 100.33) (width 0.25) (layer F.Cu) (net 16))
 (segment (start 134.62 104.14) (end 134.62 109.22) (width 0.25) (layer F.Cu) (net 24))
 (segment (start 133.35 100.33) (end 134.62 101.6) (width 0.25) (layer F.Cu) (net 14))
 (segment (start 133.35 97.79) (end 133.35 100.33) (width 0.25) (layer F.Cu) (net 14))
 (segment (start 161.29 104.14) (end 161.29 109.22) (width 0.25) (layer F.Cu) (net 23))
 (segment (start 160.025199 100.335199) (end 161.29 101.6) (width 0.25) (layer F.Cu) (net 12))
 (segment (start 140.975199 100.335199) (end 160.025199 100.335199) (width 0.25) (layer F.Cu) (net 12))
 (segment (start 138.43 97.79) (end 140.975199 100.335199) (width 0.25) (layer F.Cu) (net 12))
 (segment (start 179.07 104.14) (end 179.07 109.22) (width 0.25) (layer F.Cu) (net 22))
 (segment (start 153.67 97.79) (end 154.94 99.06) (width 0.25) (layer F.Cu) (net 10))
 (segment (start 176.53 99.06) (end 179.07 101.6) (width 0.25) (layer F.Cu) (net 10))
 (segment (start 154.94 99.06) (end 176.53 99.06) (width 0.25) (layer F.Cu) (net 10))
 (segment (start 125.73 109.22) (end 125.73 104.14) (width 0.25) (layer F.Cu) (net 21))
 (segment (start 127 101.6) (end 125.73 101.6) (width 0.25) (layer F.Cu) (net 15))
 (segment (start 130.81 97.79) (end 127 101.6) (width 0.25) (layer F.Cu) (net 15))
 (segment (start 143.51 104.14) (end 143.51 109.22) (width 0.25) (layer F.Cu) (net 20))
 (segment (start 139.7 101.6) (end 143.51 101.6) (width 0.25) (layer F.Cu) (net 13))
 (segment (start 135.89 97.79) (end 139.7 101.6) (width 0.25) (layer F.Cu) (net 13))
 (segment (start 170.18 104.14) (end 170.18 109.22) (width 0.25) (layer F.Cu) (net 19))
 (segment (start 151.13 97.79) (end 153.225189 99.885189) (width 0.25) (layer F.Cu) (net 11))
 (segment (start 168.465189 99.885189) (end 170.18 101.6) (width 0.25) (layer F.Cu) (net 11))
 (segment (start 153.225189 99.885189) (end 168.465189 99.885189) (width 0.25) (layer F.Cu) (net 11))
 (segment (start 187.96 104.14) (end 187.96 109.22) (width 0.25) (layer F.Cu) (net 18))
 (segment (start 184.96999 98.60999) (end 187.96 101.6) (width 0.25) (layer F.Cu) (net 9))
 (segment (start 168.108528 98.60999) (end 184.96999 98.60999) (width 0.25) (layer F.Cu) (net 9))
 (segment (start 166.150737 96.652199) (end 168.108528 98.60999) (width 0.25) (layer F.Cu) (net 9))
 (segment (start 157.347801 96.652199) (end 166.150737 96.652199) (width 0.25) (layer F.Cu) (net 9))
 (segment (start 156.21 97.79) (end 157.347801 96.652199) (width 0.25) (layer F.Cu) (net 9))
 (segment (start 125.73 94.8182) (end 121.6406 90.7288) (width 0.25) (layer F.Cu) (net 17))
 (segment (start 125.73 97.79) (end 125.73 94.8182) (width 0.25) (layer F.Cu) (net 17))
 (segment (start 121.92 90.4494) (end 121.6406 90.7288) (width 0.25) (layer F.Cu) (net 17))
 (segment (start 121.92 86.36) (end 121.92 90.4494) (width 0.25) (layer F.Cu) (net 17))
 (segment (start 216.895799 107.386001) (end 218.1606 106.1212) (width 0.25) (layer B.Cu) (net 8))
 (segment (start 170.848094 97.79) (end 180.444095 107.386001) (width 0.25) (layer B.Cu) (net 8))
 (segment (start 158.75 97.79) (end 170.848094 97.79) (width 0.25) (layer B.Cu) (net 8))
 (segment (start 207.01 104.902) (end 204.525999 107.386001) (width 0.25) (layer B.Cu) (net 8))
 (segment (start 207.01 102.87) (end 207.01 104.902) (width 0.25) (layer B.Cu) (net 8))
 (segment (start 204.525999 107.386001) (end 216.895799 107.386001) (width 0.25) (layer B.Cu) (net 8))
 (segment (start 180.444095 107.386001) (end 204.525999 107.386001) (width 0.25) (layer B.Cu) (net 8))
 (segment (start 89.8906 102.87) (end 97.79 102.87) (width 0.25) (layer F.Cu) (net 7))
 (segment (start 86.6394 99.6188) (end 89.8906 102.87) (width 0.25) (layer F.Cu) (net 7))
 (segment (start 157.612199 89.032199) (end 158.75 90.17) (width 0.25) (layer B.Cu) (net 7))
 (segment (start 150.829457 89.032199) (end 157.612199 89.032199) (width 0.25) (layer B.Cu) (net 7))
 (segment (start 150.379448 88.58219) (end 150.829457 89.032199) (width 0.25) (layer B.Cu) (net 7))
 (segment (start 112.07781 88.58219) (end 150.379448 88.58219) (width 0.25) (layer B.Cu) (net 7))
 (segment (start 97.79 102.87) (end 112.07781 88.58219) (width 0.25) (layer B.Cu) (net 7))
 (segment (start 201.2188 106.1212) (end 187.96 119.38) (width 0.25) (layer F.Cu) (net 1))
 (segment (start 213.6394 106.1212) (end 201.2188 106.1212) (width 0.25) (layer F.Cu) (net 1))
 (segment (start 118.816001 89.032199) (end 117.1194 90.7288) (width 0.25) (layer B.Cu) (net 1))
 (segment (start 139.832199 89.032199) (end 118.816001 89.032199) (width 0.25) (layer B.Cu) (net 1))
 (segment (start 140.97 90.17) (end 139.832199 89.032199) (width 0.25) (layer B.Cu) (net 1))
 (segment (start 110.9218 119.38) (end 91.1606 99.6188) (width 0.25) (layer B.Cu) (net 1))
 (segment (start 116.84 119.38) (end 110.9218 119.38) (width 0.25) (layer B.Cu) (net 1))
 (segment (start 117.1194 90.7288) (end 100.0506 90.7288) (width 0.25) (layer F.Cu) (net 1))
 (segment (start 100.0506 90.7288) (end 91.1606 99.6188) (width 0.25) (layer F.Cu) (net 1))
 (segment (start 167.64 95.25) (end 167.64 96.43872) (width 0.25) (layer F.Cu) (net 5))
 (segment (start 176.53 86.36) (end 167.64 95.25) (width 0.25) (layer F.Cu) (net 5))
 (segment (start 193.04 102.87) (end 196.85 102.87) (width 0.25) (layer B.Cu) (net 5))
 (segment (start 176.53 86.36) (end 193.04 102.87) (width 0.25) (layer B.Cu) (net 5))
 (segment (start 125.73 90.492506) (end 125.73 90.17) (width 0.25) (layer B.Cu) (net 5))
 (segment (start 113.352506 102.87) (end 125.73 90.492506) (width 0.25) (layer B.Cu) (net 5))
 (segment (start 107.95 102.87) (end 113.352506 102.87) (width 0.25) (layer B.Cu) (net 5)))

